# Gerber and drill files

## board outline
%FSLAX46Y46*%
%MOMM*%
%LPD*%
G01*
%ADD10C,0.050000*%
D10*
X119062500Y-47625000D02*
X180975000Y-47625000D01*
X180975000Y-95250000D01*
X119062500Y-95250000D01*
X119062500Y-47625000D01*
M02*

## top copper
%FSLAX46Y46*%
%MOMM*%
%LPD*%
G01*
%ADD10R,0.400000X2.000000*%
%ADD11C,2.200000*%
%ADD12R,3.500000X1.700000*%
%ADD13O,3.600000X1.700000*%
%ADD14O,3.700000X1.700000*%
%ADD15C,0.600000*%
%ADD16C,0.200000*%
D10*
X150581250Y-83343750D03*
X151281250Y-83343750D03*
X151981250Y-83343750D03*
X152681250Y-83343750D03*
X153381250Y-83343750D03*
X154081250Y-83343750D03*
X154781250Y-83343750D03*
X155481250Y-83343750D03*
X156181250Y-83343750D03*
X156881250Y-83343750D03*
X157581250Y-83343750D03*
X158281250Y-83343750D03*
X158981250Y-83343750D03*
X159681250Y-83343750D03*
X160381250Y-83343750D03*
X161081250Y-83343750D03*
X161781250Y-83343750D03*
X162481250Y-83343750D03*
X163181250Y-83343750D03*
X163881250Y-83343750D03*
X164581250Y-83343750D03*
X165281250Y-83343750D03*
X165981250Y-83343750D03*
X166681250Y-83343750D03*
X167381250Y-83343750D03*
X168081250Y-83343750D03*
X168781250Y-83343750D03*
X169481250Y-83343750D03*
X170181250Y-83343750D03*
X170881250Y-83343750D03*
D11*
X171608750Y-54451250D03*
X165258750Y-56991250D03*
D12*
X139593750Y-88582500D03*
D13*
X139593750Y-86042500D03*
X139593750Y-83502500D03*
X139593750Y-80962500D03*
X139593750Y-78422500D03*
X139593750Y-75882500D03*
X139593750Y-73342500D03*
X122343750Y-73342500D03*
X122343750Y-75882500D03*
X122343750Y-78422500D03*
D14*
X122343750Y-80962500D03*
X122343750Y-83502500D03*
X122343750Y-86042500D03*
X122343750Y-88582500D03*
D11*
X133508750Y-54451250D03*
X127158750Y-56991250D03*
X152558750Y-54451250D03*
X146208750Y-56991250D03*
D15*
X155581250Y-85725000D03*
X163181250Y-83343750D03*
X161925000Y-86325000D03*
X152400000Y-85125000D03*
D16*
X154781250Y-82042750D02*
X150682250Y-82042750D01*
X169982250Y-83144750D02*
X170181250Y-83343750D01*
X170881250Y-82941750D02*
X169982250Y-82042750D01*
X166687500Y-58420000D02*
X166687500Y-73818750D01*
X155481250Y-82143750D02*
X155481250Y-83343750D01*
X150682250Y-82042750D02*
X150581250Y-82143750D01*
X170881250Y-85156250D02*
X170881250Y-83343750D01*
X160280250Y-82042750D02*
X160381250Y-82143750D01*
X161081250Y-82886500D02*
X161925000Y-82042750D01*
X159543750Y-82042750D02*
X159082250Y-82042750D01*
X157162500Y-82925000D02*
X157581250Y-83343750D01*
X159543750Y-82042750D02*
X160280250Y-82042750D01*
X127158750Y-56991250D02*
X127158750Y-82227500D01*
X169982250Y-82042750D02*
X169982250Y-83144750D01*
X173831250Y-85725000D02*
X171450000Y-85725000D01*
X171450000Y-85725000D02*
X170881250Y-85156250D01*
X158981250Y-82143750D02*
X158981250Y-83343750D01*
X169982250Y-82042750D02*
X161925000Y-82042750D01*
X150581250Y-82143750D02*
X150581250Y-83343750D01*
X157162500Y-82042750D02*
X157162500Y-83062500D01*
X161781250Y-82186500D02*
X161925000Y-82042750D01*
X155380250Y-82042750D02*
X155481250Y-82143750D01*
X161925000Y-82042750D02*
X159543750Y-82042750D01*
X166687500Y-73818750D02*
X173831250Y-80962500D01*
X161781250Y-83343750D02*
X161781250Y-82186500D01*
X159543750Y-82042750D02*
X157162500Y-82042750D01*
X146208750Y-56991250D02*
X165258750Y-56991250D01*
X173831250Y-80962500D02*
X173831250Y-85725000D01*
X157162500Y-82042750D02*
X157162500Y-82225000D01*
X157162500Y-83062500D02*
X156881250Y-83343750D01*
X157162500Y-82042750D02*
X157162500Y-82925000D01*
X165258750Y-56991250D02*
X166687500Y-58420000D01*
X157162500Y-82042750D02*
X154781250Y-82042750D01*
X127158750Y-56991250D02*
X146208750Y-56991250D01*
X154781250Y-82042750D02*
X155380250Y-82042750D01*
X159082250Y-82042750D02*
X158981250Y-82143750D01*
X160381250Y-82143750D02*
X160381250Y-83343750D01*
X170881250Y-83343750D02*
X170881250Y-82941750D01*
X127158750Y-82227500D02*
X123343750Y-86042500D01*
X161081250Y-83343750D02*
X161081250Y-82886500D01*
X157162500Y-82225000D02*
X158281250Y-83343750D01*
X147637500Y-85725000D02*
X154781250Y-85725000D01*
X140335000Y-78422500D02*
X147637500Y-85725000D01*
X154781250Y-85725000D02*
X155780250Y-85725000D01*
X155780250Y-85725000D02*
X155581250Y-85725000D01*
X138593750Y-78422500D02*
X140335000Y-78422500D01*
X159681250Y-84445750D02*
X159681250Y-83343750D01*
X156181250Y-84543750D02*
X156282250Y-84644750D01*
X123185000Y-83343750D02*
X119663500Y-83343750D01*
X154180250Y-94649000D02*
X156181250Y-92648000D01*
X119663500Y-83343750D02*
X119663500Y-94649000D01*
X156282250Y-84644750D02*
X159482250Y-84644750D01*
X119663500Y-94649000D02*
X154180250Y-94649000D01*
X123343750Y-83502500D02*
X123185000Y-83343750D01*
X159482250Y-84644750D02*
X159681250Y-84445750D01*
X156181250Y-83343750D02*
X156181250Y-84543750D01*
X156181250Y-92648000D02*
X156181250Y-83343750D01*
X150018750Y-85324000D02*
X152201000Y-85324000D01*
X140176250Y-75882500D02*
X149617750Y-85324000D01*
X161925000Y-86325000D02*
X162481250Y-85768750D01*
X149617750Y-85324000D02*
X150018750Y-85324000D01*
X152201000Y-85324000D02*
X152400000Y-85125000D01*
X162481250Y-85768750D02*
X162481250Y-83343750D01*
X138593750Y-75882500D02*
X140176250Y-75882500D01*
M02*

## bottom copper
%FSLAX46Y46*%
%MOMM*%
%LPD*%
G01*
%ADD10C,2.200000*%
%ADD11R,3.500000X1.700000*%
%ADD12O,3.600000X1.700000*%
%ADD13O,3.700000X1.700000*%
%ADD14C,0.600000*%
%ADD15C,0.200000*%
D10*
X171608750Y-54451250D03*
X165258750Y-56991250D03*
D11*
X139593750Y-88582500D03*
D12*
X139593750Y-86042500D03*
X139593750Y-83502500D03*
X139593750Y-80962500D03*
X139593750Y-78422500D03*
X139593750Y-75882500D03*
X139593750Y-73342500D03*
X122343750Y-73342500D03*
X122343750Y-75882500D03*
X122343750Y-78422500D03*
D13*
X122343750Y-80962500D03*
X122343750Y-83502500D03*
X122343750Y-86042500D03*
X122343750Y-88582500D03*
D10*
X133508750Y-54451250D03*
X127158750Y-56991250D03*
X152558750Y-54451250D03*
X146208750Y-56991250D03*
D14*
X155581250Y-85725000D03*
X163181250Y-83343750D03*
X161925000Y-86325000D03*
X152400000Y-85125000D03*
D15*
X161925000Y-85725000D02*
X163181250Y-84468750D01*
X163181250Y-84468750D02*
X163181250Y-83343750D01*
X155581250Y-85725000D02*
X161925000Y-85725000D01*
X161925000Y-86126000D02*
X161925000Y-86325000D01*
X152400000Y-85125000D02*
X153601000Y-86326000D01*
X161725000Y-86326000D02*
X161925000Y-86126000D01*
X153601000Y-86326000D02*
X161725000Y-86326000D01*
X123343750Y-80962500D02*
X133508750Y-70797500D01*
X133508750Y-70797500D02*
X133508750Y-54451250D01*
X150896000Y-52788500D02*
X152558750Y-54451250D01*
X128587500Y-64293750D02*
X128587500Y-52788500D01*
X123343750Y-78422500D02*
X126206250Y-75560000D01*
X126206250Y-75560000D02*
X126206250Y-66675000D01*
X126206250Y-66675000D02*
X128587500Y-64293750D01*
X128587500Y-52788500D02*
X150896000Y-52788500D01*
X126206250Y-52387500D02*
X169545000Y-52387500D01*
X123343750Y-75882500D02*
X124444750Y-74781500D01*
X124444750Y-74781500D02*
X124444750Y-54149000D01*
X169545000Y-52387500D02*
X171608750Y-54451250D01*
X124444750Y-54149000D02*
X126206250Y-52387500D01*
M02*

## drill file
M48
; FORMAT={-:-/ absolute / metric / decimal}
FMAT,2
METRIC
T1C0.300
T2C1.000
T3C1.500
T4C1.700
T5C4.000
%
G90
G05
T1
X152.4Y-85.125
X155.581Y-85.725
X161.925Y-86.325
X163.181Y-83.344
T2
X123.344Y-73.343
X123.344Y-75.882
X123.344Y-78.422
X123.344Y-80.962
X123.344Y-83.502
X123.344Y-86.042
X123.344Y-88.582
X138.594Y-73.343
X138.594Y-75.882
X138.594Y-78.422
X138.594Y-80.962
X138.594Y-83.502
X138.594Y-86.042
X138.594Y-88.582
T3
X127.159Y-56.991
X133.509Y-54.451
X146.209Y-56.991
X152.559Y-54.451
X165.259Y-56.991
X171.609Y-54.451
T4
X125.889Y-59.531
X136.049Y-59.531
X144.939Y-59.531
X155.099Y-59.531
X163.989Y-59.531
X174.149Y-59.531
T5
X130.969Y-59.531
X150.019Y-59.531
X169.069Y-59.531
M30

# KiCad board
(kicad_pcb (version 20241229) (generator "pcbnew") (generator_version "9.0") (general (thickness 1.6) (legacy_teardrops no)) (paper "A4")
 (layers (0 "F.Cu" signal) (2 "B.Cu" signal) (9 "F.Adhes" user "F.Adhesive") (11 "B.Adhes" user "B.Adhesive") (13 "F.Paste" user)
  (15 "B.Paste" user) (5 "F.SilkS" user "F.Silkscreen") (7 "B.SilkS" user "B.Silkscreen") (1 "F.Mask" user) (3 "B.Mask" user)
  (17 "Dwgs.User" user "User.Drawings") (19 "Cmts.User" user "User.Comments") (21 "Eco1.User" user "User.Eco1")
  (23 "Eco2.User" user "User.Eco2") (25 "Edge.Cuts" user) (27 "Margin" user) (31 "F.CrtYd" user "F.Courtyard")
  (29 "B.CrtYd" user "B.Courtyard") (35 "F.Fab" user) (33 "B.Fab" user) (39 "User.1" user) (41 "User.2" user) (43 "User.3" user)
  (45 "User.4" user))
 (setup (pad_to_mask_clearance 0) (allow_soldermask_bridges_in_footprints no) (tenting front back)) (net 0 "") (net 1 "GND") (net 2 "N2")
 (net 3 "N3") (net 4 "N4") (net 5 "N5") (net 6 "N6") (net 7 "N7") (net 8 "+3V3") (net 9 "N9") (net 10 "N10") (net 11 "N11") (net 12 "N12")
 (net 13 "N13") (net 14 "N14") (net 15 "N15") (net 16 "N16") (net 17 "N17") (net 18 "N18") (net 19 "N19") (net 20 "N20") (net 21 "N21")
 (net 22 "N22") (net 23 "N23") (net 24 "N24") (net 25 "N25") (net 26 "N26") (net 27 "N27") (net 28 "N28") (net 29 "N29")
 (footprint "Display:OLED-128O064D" (layer "F.Cu") (at 160.73125 83.34375)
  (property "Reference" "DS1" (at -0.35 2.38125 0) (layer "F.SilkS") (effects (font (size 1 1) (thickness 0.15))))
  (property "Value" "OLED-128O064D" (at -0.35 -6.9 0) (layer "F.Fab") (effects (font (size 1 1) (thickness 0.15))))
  (pad "1" smd rect (at -10.15 0) (size 0.4 2) (layers "F.Cu" "F.Mask" "F.Paste") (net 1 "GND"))
  (pad "2" smd rect (at -9.45 0) (size 0.4 2) (layers "F.Cu" "F.Mask" "F.Paste") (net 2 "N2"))
  (pad "3" smd rect (at -8.75 0) (size 0.4 2) (layers "F.Cu" "F.Mask" "F.Paste") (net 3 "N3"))
  (pad "4" smd rect (at -8.05 0) (size 0.4 2) (layers "F.Cu" "F.Mask" "F.Paste") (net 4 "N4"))
  (pad "5" smd rect (at -7.35 0) (size 0.4 2) (layers "F.Cu" "F.Mask" "F.Paste") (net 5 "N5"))
  (pad "6" smd rect (at -6.65 0) (size 0.4 2) (layers "F.Cu" "F.Mask" "F.Paste") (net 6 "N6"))
  (pad "7" smd rect (at -5.95 0) (size 0.4 2) (layers "F.Cu" "F.Mask" "F.Paste") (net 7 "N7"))
  (pad "8" smd rect (at -5.25 0) (size 0.4 2) (layers "F.Cu" "F.Mask" "F.Paste") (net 1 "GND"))
  (pad "9" smd rect (at -4.55 0) (size 0.4 2) (layers "F.Cu" "F.Mask" "F.Paste") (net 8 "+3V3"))
  (pad "10" smd rect (at -3.85 0) (size 0.4 2) (layers "F.Cu" "F.Mask" "F.Paste") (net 1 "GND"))
  (pad "11" smd rect (at -3.15 0) (size 0.4 2) (layers "F.Cu" "F.Mask" "F.Paste") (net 1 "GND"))
  (pad "12" smd rect (at -2.45 0) (size 0.4 2) (layers "F.Cu" "F.Mask" "F.Paste") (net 1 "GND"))
  (pad "13" smd rect (at -1.75 0) (size 0.4 2) (layers "F.Cu" "F.Mask" "F.Paste") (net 1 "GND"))
  (pad "14" smd rect (at -1.05 0) (size 0.4 2) (layers "F.Cu" "F.Mask" "F.Paste") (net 8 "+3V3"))
  (pad "15" smd rect (at -0.35 0) (size 0.4 2) (layers "F.Cu" "F.Mask" "F.Paste") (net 1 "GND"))
  (pad "16" smd rect (at 0.35 0) (size 0.4 2) (layers "F.Cu" "F.Mask" "F.Paste") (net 1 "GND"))
  (pad "17" smd rect (at 1.05 0) (size 0.4 2) (layers "F.Cu" "F.Mask" "F.Paste") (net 1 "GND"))
  (pad "18" smd rect (at 1.75 0) (size 0.4 2) (layers "F.Cu" "F.Mask" "F.Paste") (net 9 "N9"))
  (pad "19" smd rect (at 2.45 0) (size 0.4 2) (layers "F.Cu" "F.Mask" "F.Paste") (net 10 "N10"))
  (pad "20" smd rect (at 3.15 0) (size 0.4 2) (layers "F.Cu" "F.Mask" "F.Paste") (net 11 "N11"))
  (pad "21" smd rect (at 3.85 0) (size 0.4 2) (layers "F.Cu" "F.Mask" "F.Paste") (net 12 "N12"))
  (pad "22" smd rect (at 4.55 0) (size 0.4 2) (layers "F.Cu" "F.Mask" "F.Paste") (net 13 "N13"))
  (pad "23" smd rect (at 5.25 0) (size 0.4 2) (layers "F.Cu" "F.Mask" "F.Paste") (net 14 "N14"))
  (pad "24" smd rect (at 5.95 0) (size 0.4 2) (layers "F.Cu" "F.Mask" "F.Paste") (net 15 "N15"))
  (pad "25" smd rect (at 6.65 0) (size 0.4 2) (layers "F.Cu" "F.Mask" "F.Paste") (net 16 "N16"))
  (pad "26" smd rect (at 7.35 0) (size 0.4 2) (layers "F.Cu" "F.Mask" "F.Paste") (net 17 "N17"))
  (pad "27" smd rect (at 8.05 0) (size 0.4 2) (layers "F.Cu" "F.Mask" "F.Paste") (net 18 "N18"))
  (pad "28" smd rect (at 8.75 0) (size 0.4 2) (layers "F.Cu" "F.Mask" "F.Paste") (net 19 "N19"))
  (pad "29" smd rect (at 9.45 0) (size 0.4 2) (layers "F.Cu" "F.Mask" "F.Paste") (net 1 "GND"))
  (pad "30" smd rect (at 10.15 0) (size 0.4 2) (layers "F.Cu" "F.Mask" "F.Paste") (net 1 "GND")))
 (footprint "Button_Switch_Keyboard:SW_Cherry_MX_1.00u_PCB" (layer "F.Cu") (at 171.60875 54.45125)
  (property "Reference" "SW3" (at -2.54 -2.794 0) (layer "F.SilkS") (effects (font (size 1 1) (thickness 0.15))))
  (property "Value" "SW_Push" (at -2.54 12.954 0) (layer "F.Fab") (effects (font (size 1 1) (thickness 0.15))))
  (pad "" np_thru_hole circle (at -7.62 5.08) (size 1.7 1.7) (drill 1.7) (layers "*.Cu" "*.Mask"))
  (pad "" np_thru_hole circle (at -2.54 5.08) (size 4 4) (drill 4) (layers "*.Cu" "*.Mask"))
  (pad "" np_thru_hole circle (at 2.54 5.08) (size 1.7 1.7) (drill 1.7) (layers "*.Cu" "*.Mask"))
  (pad "1" thru_hole circle (at 0 0) (size 2.2 2.2) (drill 1.5) (layers "*.Cu" "*.Mask") (remove_unused_layers no) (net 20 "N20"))
  (pad "2" thru_hole circle (at -6.35 2.54) (size 2.2 2.2) (drill 1.5) (layers "*.Cu" "*.Mask") (remove_unused_layers no) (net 1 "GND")))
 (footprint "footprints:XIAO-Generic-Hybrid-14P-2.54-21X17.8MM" (layer "F.Cu") (at 130.96875 80.9625 180)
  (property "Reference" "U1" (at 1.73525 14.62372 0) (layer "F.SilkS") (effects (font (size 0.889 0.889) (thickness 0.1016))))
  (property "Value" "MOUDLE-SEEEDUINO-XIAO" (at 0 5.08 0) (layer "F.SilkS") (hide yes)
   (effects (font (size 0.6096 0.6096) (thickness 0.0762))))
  (pad "1" thru_hole rect (at -7.625 -7.62 180) (size 3.5 1.7) (drill 1 (offset -1 0)) (layers "*.Cu" "*.Mask") (remove_unused_layers no)
   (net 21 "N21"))
  (pad "2" thru_hole oval (at -7.625 -5.08 180) (size 3.6 1.7) (drill 1 (offset -1 0)) (layers "*.Cu" "*.Mask") (remove_unused_layers no)
   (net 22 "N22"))
  (pad "3" thru_hole oval (at -7.625 -2.54 180) (size 3.6 1.7) (drill 1 (offset -1 0)) (layers "*.Cu" "*.Mask") (remove_unused_layers no)
   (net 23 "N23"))
  (pad "4" thru_hole oval (at -7.625 0 180) (size 3.6 1.7) (drill 1 (offset -1 0)) (layers "*.Cu" "*.Mask") (remove_unused_layers no)
   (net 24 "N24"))
  (pad "5" thru_hole oval (at -7.625 2.54 180) (size 3.6 1.7) (drill 1 (offset -1 0)) (layers "*.Cu" "*.Mask") (remove_unused_layers no)
   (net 10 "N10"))
  (pad "6" thru_hole oval (at -7.625 5.08) (size 3.6 1.7) (drill 1 (offset 1 0)) (layers "*.Cu" "*.Mask") (remove_unused_layers no)
   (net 9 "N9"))
  (pad "7" thru_hole oval (at -7.625 7.62 180) (size 3.6 1.7) (drill 1 (offset -1 0)) (layers "*.Cu" "*.Mask") (remove_unused_layers no)
   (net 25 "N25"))
  (pad "8" thru_hole oval (at 7.625 7.62 180) (size 3.6 1.7) (drill 1 (offset 1 0)) (layers "*.Cu" "*.Mask") (remove_unused_layers no)
   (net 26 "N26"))
  (pad "9" thru_hole oval (at 7.625 5.08 180) (size 3.6 1.7) (drill 1 (offset 1 0)) (layers "*.Cu" "*.Mask") (remove_unused_layers no)
   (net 20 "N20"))
  (pad "10" thru_hole oval (at 7.625 2.54 180) (size 3.6 1.7) (drill 1 (offset 1 0)) (layers "*.Cu" "*.Mask") (remove_unused_layers no)
   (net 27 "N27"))
  (pad "11" thru_hole oval (at 7.625 0 180) (size 3.7 1.7) (drill 1 (offset 1 0)) (layers "*.Cu" "*.Mask") (remove_unused_layers no)
   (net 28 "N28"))
  (pad "12" thru_hole oval (at 7.625 -2.54 180) (size 3.7 1.7) (drill 1 (offset 1 0)) (layers "*.Cu" "*.Mask") (remove_unused_layers no)
   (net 8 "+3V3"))
  (pad "13" thru_hole oval (at 7.625 -5.08 180) (size 3.7 1.7) (drill 1 (offset 1 0)) (layers "*.Cu" "*.Mask") (remove_unused_layers no)
   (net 1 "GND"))
  (pad "14" thru_hole oval (at 7.625 -7.62 180) (size 3.7 1.7) (drill 1 (offset 1 0)) (layers "*.Cu" "*.Mask") (remove_unused_layers no)
   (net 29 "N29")))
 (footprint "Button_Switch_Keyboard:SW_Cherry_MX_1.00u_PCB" (layer "F.Cu") (at 133.50875 54.45125)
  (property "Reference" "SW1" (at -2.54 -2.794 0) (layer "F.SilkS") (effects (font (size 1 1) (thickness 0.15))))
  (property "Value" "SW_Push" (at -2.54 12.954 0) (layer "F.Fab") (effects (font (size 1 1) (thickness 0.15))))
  (pad "" np_thru_hole circle (at -7.62 5.08) (size 1.7 1.7) (drill 1.7) (layers "*.Cu" "*.Mask"))
  (pad "" np_thru_hole circle (at -2.54 5.08) (size 4 4) (drill 4) (layers "*.Cu" "*.Mask"))
  (pad "" np_thru_hole circle (at 2.54 5.08) (size 1.7 1.7) (drill 1.7) (layers "*.Cu" "*.Mask"))
  (pad "1" thru_hole circle (at 0 0) (size 2.2 2.2) (drill 1.5) (layers "*.Cu" "*.Mask") (remove_unused_layers no) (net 28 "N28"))
  (pad "2" thru_hole circle (at -6.35 2.54) (size 2.2 2.2) (drill 1.5) (layers "*.Cu" "*.Mask") (remove_unused_layers no) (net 1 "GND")))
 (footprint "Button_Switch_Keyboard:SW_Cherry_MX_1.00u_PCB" (layer "F.Cu") (at 152.55875 54.45125)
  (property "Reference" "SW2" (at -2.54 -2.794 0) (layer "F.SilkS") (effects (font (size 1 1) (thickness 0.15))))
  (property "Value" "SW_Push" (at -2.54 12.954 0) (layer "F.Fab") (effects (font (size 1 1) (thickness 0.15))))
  (pad "" np_thru_hole circle (at -7.62 5.08) (size 1.7 1.7) (drill 1.7) (layers "*.Cu" "*.Mask"))
  (pad "" np_thru_hole circle (at -2.54 5.08) (size 4 4) (drill 4) (layers "*.Cu" "*.Mask"))
  (pad "" np_thru_hole circle (at 2.54 5.08) (size 1.7 1.7) (drill 1.7) (layers "*.Cu" "*.Mask"))
  (pad "1" thru_hole circle (at 0 0) (size 2.2 2.2) (drill 1.5) (layers "*.Cu" "*.Mask") (remove_unused_layers no) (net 27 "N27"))
  (pad "2" thru_hole circle (at -6.35 2.54) (size 2.2 2.2) (drill 1.5) (layers "*.Cu" "*.Mask") (remove_unused_layers no) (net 1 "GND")))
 (gr_rect (start 119.0625 47.625) (end 180.975 95.25) (stroke (width 0.05) (type default)) (fill no) (layer "Edge.Cuts"))
 (segment (start 154.78125 82.04275) (end 150.68225 82.04275) (width 0.2) (layer "F.Cu") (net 1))
 (segment (start 169.98225 83.14475) (end 170.18125 83.34375) (width 0.2) (layer "F.Cu") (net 1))
 (segment (start 170.88125 82.94175) (end 169.98225 82.04275) (width 0.2) (layer "F.Cu") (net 1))
 (segment (start 166.6875 58.42) (end 166.6875 73.81875) (width 0.2) (layer "F.Cu") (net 1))
 (segment (start 155.48125 82.14375) (end 155.48125 83.34375) (width 0.2) (layer "F.Cu") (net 1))
 (segment (start 150.68225 82.04275) (end 150.58125 82.14375) (width 0.2) (layer "F.Cu") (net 1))
 (segment (start 170.88125 85.15625) (end 170.88125 83.34375) (width 0.2) (layer "F.Cu") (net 1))
 (segment (start 160.28025 82.04275) (end 160.38125 82.14375) (width 0.2) (layer "F.Cu") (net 1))
 (segment (start 161.08125 82.8865) (end 161.925 82.04275) (width 0.2) (layer "F.Cu") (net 1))
 (segment (start 159.54375 82.04275) (end 159.08225 82.04275) (width 0.2) (layer "F.Cu") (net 1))
 (segment (start 157.1625 82.925) (end 157.58125 83.34375) (width 0.2) (layer "F.Cu") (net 1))
 (segment (start 159.54375 82.04275) (end 160.28025 82.04275) (width 0.2) (layer "F.Cu") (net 1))
 (segment (start 127.15875 56.99125) (end 127.15875 82.2275) (width 0.2) (layer "F.Cu") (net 1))
 (segment (start 169.98225 82.04275) (end 169.98225 83.14475) (width 0.2) (layer "F.Cu") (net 1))
 (segment (start 173.83125 85.725) (end 171.45 85.725) (width 0.2) (layer "F.Cu") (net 1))
 (segment (start 171.45 85.725) (end 170.88125 85.15625) (width 0.2) (layer "F.Cu") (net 1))
 (segment (start 158.98125 82.14375) (end 158.98125 83.34375) (width 0.2) (layer "F.Cu") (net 1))
 (segment (start 169.98225 82.04275) (end 161.925 82.04275) (width 0.2) (layer "F.Cu") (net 1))
 (segment (start 150.58125 82.14375) (end 150.58125 83.34375) (width 0.2) (layer "F.Cu") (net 1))
 (segment (start 157.1625 82.04275) (end 157.1625 83.0625) (width 0.2) (layer "F.Cu") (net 1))
 (segment (start 161.78125 82.1865) (end 161.925 82.04275) (width 0.2) (layer "F.Cu") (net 1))
 (segment (start 155.38025 82.04275) (end 155.48125 82.14375) (width 0.2) (layer "F.Cu") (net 1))
 (segment (start 161.925 82.04275) (end 159.54375 82.04275) (width 0.2) (layer "F.Cu") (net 1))
 (segment (start 166.6875 73.81875) (end 173.83125 80.9625) (width 0.2) (layer "F.Cu") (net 1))
 (segment (start 161.78125 83.34375) (end 161.78125 82.1865) (width 0.2) (layer "F.Cu") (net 1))
 (segment (start 159.54375 82.04275) (end 157.1625 82.04275) (width 0.2) (layer "F.Cu") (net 1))
 (segment (start 146.20875 56.99125) (end 165.25875 56.99125) (width 0.2) (layer "F.Cu") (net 1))
 (segment (start 173.83125 80.9625) (end 173.83125 85.725) (width 0.2) (layer "F.Cu") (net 1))
 (segment (start 157.1625 82.04275) (end 157.1625 82.225) (width 0.2) (layer "F.Cu") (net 1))
 (segment (start 157.1625 83.0625) (end 156.88125 83.34375) (width 0.2) (layer "F.Cu") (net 1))
 (segment (start 157.1625 82.04275) (end 157.1625 82.925) (width 0.2) (layer "F.Cu") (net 1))
 (segment (start 165.25875 56.99125) (end 166.6875 58.42) (width 0.2) (layer "F.Cu") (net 1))
 (segment (start 157.1625 82.04275) (end 154.78125 82.04275) (width 0.2) (layer "F.Cu") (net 1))
 (segment (start 127.15875 56.99125) (end 146.20875 56.99125) (width 0.2) (layer "F.Cu") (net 1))
 (segment (start 154.78125 82.04275) (end 155.38025 82.04275) (width 0.2) (layer "F.Cu") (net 1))
 (segment (start 159.08225 82.04275) (end 158.98125 82.14375) (width 0.2) (layer "F.Cu") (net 1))
 (segment (start 160.38125 82.14375) (end 160.38125 83.34375) (width 0.2) (layer "F.Cu") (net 1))
 (segment (start 170.88125 83.34375) (end 170.88125 82.94175) (width 0.2) (layer "F.Cu") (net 1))
 (segment (start 127.15875 82.2275) (end 123.34375 86.0425) (width 0.2) (layer "F.Cu") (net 1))
 (segment (start 161.08125 83.34375) (end 161.08125 82.8865) (width 0.2) (layer "F.Cu") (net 1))
 (segment (start 157.1625 82.225) (end 158.28125 83.34375) (width 0.2) (layer "F.Cu") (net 1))
 (segment (start 147.6375 85.725) (end 154.78125 85.725) (width 0.2) (layer "F.Cu") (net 10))
 (segment (start 140.335 78.4225) (end 147.6375 85.725) (width 0.2) (layer "F.Cu") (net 10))
 (segment (start 154.78125 85.725) (end 155.78025 85.725) (width 0.2) (layer "F.Cu") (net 10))
 (segment (start 155.78025 85.725) (end 155.58125 85.725) (width 0.2) (layer "F.Cu") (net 10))
 (segment (start 138.59375 78.4225) (end 140.335 78.4225) (width 0.2) (layer "F.Cu") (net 10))
 (via (at 155.58125 85.725) (size 0.6) (drill 0.3) (layers "F.Cu" "B.Cu") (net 10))
 (via (at 163.18125 83.34375) (size 0.6) (drill 0.3) (layers "F.Cu" "B.Cu") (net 10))
 (segment (start 161.925 85.725) (end 163.18125 84.46875) (width 0.2) (layer "B.Cu") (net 10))
 (segment (start 163.18125 84.46875) (end 163.18125 83.34375) (width 0.2) (layer "B.Cu") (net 10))
 (segment (start 155.58125 85.725) (end 161.925 85.725) (width 0.2) (layer "B.Cu") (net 10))
 (segment (start 159.68125 84.44575) (end 159.68125 83.34375) (width 0.2) (layer "F.Cu") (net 8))
 (segment (start 156.18125 84.54375) (end 156.28225 84.64475) (width 0.2) (layer "F.Cu") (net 8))
 (segment (start 123.185 83.34375) (end 119.6635 83.34375) (width 0.2) (layer "F.Cu") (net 8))
 (segment (start 154.18025 94.649) (end 156.18125 92.648) (width 0.2) (layer "F.Cu") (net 8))
 (segment (start 119.6635 83.34375) (end 119.6635 94.649) (width 0.2) (layer "F.Cu") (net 8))
 (segment (start 156.28225 84.64475) (end 159.48225 84.64475) (width 0.2) (layer "F.Cu") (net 8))
 (segment (start 119.6635 94.649) (end 154.18025 94.649) (width 0.2) (layer "F.Cu") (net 8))
 (segment (start 123.34375 83.5025) (end 123.185 83.34375) (width 0.2) (layer "F.Cu") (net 8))
 (segment (start 159.48225 84.64475) (end 159.68125 84.44575) (width 0.2) (layer "F.Cu") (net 8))
 (segment (start 156.18125 83.34375) (end 156.18125 84.54375) (width 0.2) (layer "F.Cu") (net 8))
 (segment (start 156.18125 92.648) (end 156.18125 83.34375) (width 0.2) (layer "F.Cu") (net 8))
 (segment (start 150.01875 85.324) (end 152.201 85.324) (width 0.2) (layer "F.Cu") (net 9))
 (segment (start 140.17625 75.8825) (end 149.61775 85.324) (width 0.2) (layer "F.Cu") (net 9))
 (segment (start 161.925 86.325) (end 162.48125 85.76875) (width 0.2) (layer "F.Cu") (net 9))
 (segment (start 149.61775 85.324) (end 150.01875 85.324) (width 0.2) (layer "F.Cu") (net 9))
 (segment (start 152.201 85.324) (end 152.4 85.125) (width 0.2) (layer "F.Cu") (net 9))
 (segment (start 162.48125 85.76875) (end 162.48125 83.34375) (width 0.2) (layer "F.Cu") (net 9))
 (segment (start 138.59375 75.8825) (end 140.17625 75.8825) (width 0.2) (layer "F.Cu") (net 9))
 (via (at 161.925 86.325) (size 0.6) (drill 0.3) (layers "F.Cu" "B.Cu") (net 9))
 (via (at 152.4 85.125) (size 0.6) (drill 0.3) (layers "F.Cu" "B.Cu") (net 9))
 (segment (start 161.925 86.126) (end 161.925 86.325) (width 0.2) (layer "B.Cu") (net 9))
 (segment (start 152.4 85.125) (end 153.601 86.326) (width 0.2) (layer "B.Cu") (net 9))
 (segment (start 161.725 86.326) (end 161.925 86.126) (width 0.2) (layer "B.Cu") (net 9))
 (segment (start 153.601 86.326) (end 161.725 86.326) (width 0.2) (layer "B.Cu") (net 9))
 (segment (start 123.34375 80.9625) (end 133.50875 70.7975) (width 0.2) (layer "B.Cu") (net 28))
 (segment (start 133.50875 70.7975) (end 133.50875 54.45125) (width 0.2) (layer "B.Cu") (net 28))
 (segment (start 150.896 52.7885) (end 152.55875 54.45125) (width 0.2) (layer "B.Cu") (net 27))
 (segment (start 128.5875 64.29375) (end 128.5875 52.7885) (width 0.2) (layer "B.Cu") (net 27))
 (segment (start 123.34375 78.4225) (end 126.20625 75.56) (width 0.2) (layer "B.Cu") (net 27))
 (segment (start 126.20625 75.56) (end 126.20625 66.675) (width 0.2) (layer "B.Cu") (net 27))
 (segment (start 126.20625 66.675) (end 128.5875 64.29375) (width 0.2) (layer "B.Cu") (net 27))
 (segment (start 128.5875 52.7885) (end 150.896 52.7885) (width 0.2) (layer "B.Cu") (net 27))
 (segment (start 126.20625 52.3875) (end 169.545 52.3875) (width 0.2) (layer "B.Cu") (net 20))
 (segment (start 123.34375 75.8825) (end 124.44475 74.7815) (width 0.2) (layer "B.Cu") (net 20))
 (segment (start 124.44475 74.7815) (end 124.44475 54.149) (width 0.2) (layer "B.Cu") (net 20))
 (segment (start 169.545 52.3875) (end 171.60875 54.45125) (width 0.2) (layer "B.Cu") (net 20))
 (segment (start 124.44475 54.149) (end 126.20625 52.3875) (width 0.2) (layer "B.Cu") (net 20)))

